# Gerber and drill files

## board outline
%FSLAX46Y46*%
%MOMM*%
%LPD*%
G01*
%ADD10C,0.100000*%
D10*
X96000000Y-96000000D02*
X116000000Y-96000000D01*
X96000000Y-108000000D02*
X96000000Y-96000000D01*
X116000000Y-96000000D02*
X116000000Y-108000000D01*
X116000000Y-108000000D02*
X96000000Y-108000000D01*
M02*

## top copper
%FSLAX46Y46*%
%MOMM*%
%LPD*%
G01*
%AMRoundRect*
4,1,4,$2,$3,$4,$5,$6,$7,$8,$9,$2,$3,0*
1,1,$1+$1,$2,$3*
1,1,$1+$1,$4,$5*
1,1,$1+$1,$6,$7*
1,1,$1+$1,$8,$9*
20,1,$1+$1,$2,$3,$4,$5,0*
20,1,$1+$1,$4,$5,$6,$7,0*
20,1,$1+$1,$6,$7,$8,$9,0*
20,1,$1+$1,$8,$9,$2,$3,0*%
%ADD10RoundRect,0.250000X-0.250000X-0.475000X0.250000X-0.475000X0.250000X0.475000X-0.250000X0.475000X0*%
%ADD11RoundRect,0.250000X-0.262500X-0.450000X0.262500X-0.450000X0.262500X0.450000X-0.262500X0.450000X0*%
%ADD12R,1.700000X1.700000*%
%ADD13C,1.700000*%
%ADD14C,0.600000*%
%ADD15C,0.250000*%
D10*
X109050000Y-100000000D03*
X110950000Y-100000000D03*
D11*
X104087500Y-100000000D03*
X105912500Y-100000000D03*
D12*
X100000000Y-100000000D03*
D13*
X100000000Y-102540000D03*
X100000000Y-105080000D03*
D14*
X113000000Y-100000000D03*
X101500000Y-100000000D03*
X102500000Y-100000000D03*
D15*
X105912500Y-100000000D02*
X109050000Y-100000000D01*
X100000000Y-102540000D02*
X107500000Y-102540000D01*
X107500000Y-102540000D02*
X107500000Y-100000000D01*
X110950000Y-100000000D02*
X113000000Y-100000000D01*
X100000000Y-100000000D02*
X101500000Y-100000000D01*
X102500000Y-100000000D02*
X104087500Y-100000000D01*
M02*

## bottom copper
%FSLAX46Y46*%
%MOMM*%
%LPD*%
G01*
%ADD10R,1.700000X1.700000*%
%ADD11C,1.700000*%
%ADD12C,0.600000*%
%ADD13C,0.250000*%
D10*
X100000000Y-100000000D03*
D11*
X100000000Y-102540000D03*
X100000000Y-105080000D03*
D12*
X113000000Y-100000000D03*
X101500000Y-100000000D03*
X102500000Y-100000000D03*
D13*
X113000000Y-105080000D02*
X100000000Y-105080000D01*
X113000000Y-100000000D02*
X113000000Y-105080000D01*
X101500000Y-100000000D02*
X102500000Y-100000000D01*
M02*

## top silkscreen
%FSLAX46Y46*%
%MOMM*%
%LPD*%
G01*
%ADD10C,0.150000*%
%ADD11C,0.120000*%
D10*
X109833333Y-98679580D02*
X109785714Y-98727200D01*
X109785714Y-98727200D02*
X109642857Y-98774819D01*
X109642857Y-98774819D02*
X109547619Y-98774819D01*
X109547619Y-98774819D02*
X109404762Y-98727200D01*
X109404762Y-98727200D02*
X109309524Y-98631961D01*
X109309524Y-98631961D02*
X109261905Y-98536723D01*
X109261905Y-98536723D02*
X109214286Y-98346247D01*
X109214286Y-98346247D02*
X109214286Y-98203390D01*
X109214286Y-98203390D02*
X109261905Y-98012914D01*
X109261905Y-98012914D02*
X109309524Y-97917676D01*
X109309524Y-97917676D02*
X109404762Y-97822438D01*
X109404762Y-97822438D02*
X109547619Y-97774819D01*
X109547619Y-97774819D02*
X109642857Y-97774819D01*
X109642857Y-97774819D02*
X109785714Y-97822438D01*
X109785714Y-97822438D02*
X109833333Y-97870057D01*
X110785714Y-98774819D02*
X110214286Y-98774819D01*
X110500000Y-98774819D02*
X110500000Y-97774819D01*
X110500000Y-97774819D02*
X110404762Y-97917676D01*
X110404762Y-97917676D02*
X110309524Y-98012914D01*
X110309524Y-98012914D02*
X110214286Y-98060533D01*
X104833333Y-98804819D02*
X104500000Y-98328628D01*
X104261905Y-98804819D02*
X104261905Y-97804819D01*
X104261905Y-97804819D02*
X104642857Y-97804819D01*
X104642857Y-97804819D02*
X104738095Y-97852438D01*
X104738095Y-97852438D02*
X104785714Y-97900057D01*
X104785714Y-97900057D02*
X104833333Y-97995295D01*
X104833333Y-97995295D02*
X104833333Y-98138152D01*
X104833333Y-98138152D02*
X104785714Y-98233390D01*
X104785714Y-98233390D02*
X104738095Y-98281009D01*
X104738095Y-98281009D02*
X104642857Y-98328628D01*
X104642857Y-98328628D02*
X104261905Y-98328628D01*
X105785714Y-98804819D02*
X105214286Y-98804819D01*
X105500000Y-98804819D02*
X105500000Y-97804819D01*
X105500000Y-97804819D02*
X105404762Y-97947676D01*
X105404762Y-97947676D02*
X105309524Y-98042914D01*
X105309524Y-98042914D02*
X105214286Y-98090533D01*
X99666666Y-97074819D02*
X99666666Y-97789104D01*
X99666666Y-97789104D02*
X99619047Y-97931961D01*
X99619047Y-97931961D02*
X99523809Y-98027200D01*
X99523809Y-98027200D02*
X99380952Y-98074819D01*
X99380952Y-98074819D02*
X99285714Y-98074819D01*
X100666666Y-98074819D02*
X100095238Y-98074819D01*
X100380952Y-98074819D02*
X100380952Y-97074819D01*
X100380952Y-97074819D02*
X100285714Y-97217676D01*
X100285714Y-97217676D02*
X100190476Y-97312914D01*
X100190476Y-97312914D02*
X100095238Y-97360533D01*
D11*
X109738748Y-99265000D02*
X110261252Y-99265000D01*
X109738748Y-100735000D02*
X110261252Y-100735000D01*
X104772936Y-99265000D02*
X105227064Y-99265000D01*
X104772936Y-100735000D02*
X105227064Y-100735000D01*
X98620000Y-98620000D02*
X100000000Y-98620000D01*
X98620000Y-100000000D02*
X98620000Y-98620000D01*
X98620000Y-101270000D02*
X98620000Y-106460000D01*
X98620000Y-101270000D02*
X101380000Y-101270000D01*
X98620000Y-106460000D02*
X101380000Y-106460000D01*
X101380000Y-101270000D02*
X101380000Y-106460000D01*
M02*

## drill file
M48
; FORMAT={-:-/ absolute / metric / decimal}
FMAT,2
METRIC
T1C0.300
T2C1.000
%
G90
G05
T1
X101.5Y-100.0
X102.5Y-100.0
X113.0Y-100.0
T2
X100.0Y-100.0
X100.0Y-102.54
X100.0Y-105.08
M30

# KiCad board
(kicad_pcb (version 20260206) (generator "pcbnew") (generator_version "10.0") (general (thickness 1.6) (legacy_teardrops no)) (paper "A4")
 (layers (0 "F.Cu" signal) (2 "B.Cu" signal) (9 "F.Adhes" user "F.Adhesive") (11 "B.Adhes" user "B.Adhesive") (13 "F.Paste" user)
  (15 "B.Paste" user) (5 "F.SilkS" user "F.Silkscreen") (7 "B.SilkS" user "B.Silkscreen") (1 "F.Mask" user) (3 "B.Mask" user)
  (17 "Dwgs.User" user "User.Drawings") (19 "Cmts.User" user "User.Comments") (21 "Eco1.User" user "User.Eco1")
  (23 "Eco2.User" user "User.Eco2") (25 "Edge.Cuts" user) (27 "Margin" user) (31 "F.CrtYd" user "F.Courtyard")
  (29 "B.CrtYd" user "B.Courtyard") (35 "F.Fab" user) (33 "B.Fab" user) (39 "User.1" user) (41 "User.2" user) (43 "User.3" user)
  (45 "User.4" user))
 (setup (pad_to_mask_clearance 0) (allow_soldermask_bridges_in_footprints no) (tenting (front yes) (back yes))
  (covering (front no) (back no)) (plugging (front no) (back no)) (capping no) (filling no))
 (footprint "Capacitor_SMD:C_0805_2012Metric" (layer "F.Cu") (at 110 100)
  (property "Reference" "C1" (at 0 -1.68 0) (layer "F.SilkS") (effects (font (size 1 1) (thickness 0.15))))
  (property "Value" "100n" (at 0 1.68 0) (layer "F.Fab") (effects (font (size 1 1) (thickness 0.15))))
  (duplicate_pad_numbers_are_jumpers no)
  (fp_line (start -0.261252 -0.735) (end 0.261252 -0.735) (stroke (width 0.12) (type solid)) (layer "F.SilkS"))
  (fp_line (start -0.261252 0.735) (end 0.261252 0.735) (stroke (width 0.12) (type solid)) (layer "F.SilkS"))
  (pad "1" smd roundrect (at -0.95 0) (size 1 1.45) (layers "F.Cu" "F.Mask" "F.Paste") (roundrect_rratio 0.25) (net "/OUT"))
  (pad "2" smd roundrect (at 0.95 0) (size 1 1.45) (layers "F.Cu" "F.Mask" "F.Paste") (roundrect_rratio 0.25) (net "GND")))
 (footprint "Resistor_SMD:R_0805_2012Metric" (layer "F.Cu") (at 105 100)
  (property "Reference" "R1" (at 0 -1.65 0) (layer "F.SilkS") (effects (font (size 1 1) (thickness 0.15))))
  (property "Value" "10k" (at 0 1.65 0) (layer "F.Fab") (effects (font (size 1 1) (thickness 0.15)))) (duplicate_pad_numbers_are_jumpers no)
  (fp_line (start -0.227064 -0.735) (end 0.227064 -0.735) (stroke (width 0.12) (type solid)) (layer "F.SilkS"))
  (fp_line (start -0.227064 0.735) (end 0.227064 0.735) (stroke (width 0.12) (type solid)) (layer "F.SilkS"))
  (pad "1" smd roundrect (at -0.9125 0) (size 1.025 1.4) (layers "F.Cu" "F.Mask" "F.Paste") (roundrect_rratio 0.243902) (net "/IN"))
  (pad "2" smd roundrect (at 0.9125 0) (size 1.025 1.4) (layers "F.Cu" "F.Mask" "F.Paste") (roundrect_rratio 0.243902) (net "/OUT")))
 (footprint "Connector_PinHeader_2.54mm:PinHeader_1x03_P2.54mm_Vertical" (layer "F.Cu") (at 100 100)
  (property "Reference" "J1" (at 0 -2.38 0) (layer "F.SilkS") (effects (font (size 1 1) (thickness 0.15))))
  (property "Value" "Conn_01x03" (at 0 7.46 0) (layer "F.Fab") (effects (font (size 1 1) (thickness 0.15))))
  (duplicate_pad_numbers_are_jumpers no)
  (fp_line (start -1.38 -1.38) (end 0 -1.38) (stroke (width 0.12) (type solid)) (layer "F.SilkS"))
  (fp_line (start -1.38 0) (end -1.38 -1.38) (stroke (width 0.12) (type solid)) (layer "F.SilkS"))
  (fp_line (start -1.38 1.27) (end -1.38 6.46) (stroke (width 0.12) (type solid)) (layer "F.SilkS"))
  (fp_line (start -1.38 1.27) (end 1.38 1.27) (stroke (width 0.12) (type solid)) (layer "F.SilkS"))
  (fp_line (start -1.38 6.46) (end 1.38 6.46) (stroke (width 0.12) (type solid)) (layer "F.SilkS"))
  (fp_line (start 1.38 1.27) (end 1.38 6.46) (stroke (width 0.12) (type solid)) (layer "F.SilkS"))
  (pad "1" thru_hole rect (at 0 0) (size 1.7 1.7) (drill 1) (layers "*.Cu" "*.Mask") (remove_unused_layers no) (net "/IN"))
  (pad "2" thru_hole circle (at 0 2.54) (size 1.7 1.7) (drill 1) (layers "*.Cu" "*.Mask") (remove_unused_layers no) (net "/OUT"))
  (pad "3" thru_hole circle (at 0 5.08) (size 1.7 1.7) (drill 1) (layers "*.Cu" "*.Mask") (remove_unused_layers no) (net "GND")))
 (gr_line (start 96 96) (end 116 96) (stroke (width 0.1) (type default)) (layer "Edge.Cuts"))
 (gr_line (start 96 108) (end 96 96) (stroke (width 0.1) (type default)) (layer "Edge.Cuts"))
 (gr_line (start 116 96) (end 116 108) (stroke (width 0.1) (type default)) (layer "Edge.Cuts"))
 (gr_line (start 116 108) (end 96 108) (stroke (width 0.1) (type default)) (layer "Edge.Cuts"))
 (segment (start 105.9125 100) (end 109.05 100) (width 0.25) (layer "F.Cu") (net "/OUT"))
 (segment (start 100 102.54) (end 107.5 102.54) (width 0.25) (layer "F.Cu") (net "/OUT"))
 (segment (start 107.5 102.54) (end 107.5 100) (width 0.25) (layer "F.Cu") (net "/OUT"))
 (segment (start 110.95 100) (end 113 100) (width 0.25) (layer "F.Cu") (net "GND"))
 (via (at 113 100) (size 0.6) (drill 0.3) (layers "F.Cu" "B.Cu") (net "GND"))
 (segment (start 113 105.08) (end 100 105.08) (width 0.25) (layer "B.Cu") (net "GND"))
 (segment (start 113 100) (end 113 105.08) (width 0.25) (layer "B.Cu") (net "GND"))
 (segment (start 100 100) (end 101.5 100) (width 0.25) (layer "F.Cu") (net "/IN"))
 (segment (start 102.5 100) (end 104.0875 100) (width 0.25) (layer "F.Cu") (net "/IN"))
 (via (at 101.5 100) (size 0.6) (drill 0.3) (layers "F.Cu" "B.Cu") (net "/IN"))
 (via (at 102.5 100) (size 0.6) (drill 0.3) (layers "F.Cu" "B.Cu") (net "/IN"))
 (segment (start 101.5 100) (end 102.5 100) (width 0.25) (layer "B.Cu") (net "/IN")))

